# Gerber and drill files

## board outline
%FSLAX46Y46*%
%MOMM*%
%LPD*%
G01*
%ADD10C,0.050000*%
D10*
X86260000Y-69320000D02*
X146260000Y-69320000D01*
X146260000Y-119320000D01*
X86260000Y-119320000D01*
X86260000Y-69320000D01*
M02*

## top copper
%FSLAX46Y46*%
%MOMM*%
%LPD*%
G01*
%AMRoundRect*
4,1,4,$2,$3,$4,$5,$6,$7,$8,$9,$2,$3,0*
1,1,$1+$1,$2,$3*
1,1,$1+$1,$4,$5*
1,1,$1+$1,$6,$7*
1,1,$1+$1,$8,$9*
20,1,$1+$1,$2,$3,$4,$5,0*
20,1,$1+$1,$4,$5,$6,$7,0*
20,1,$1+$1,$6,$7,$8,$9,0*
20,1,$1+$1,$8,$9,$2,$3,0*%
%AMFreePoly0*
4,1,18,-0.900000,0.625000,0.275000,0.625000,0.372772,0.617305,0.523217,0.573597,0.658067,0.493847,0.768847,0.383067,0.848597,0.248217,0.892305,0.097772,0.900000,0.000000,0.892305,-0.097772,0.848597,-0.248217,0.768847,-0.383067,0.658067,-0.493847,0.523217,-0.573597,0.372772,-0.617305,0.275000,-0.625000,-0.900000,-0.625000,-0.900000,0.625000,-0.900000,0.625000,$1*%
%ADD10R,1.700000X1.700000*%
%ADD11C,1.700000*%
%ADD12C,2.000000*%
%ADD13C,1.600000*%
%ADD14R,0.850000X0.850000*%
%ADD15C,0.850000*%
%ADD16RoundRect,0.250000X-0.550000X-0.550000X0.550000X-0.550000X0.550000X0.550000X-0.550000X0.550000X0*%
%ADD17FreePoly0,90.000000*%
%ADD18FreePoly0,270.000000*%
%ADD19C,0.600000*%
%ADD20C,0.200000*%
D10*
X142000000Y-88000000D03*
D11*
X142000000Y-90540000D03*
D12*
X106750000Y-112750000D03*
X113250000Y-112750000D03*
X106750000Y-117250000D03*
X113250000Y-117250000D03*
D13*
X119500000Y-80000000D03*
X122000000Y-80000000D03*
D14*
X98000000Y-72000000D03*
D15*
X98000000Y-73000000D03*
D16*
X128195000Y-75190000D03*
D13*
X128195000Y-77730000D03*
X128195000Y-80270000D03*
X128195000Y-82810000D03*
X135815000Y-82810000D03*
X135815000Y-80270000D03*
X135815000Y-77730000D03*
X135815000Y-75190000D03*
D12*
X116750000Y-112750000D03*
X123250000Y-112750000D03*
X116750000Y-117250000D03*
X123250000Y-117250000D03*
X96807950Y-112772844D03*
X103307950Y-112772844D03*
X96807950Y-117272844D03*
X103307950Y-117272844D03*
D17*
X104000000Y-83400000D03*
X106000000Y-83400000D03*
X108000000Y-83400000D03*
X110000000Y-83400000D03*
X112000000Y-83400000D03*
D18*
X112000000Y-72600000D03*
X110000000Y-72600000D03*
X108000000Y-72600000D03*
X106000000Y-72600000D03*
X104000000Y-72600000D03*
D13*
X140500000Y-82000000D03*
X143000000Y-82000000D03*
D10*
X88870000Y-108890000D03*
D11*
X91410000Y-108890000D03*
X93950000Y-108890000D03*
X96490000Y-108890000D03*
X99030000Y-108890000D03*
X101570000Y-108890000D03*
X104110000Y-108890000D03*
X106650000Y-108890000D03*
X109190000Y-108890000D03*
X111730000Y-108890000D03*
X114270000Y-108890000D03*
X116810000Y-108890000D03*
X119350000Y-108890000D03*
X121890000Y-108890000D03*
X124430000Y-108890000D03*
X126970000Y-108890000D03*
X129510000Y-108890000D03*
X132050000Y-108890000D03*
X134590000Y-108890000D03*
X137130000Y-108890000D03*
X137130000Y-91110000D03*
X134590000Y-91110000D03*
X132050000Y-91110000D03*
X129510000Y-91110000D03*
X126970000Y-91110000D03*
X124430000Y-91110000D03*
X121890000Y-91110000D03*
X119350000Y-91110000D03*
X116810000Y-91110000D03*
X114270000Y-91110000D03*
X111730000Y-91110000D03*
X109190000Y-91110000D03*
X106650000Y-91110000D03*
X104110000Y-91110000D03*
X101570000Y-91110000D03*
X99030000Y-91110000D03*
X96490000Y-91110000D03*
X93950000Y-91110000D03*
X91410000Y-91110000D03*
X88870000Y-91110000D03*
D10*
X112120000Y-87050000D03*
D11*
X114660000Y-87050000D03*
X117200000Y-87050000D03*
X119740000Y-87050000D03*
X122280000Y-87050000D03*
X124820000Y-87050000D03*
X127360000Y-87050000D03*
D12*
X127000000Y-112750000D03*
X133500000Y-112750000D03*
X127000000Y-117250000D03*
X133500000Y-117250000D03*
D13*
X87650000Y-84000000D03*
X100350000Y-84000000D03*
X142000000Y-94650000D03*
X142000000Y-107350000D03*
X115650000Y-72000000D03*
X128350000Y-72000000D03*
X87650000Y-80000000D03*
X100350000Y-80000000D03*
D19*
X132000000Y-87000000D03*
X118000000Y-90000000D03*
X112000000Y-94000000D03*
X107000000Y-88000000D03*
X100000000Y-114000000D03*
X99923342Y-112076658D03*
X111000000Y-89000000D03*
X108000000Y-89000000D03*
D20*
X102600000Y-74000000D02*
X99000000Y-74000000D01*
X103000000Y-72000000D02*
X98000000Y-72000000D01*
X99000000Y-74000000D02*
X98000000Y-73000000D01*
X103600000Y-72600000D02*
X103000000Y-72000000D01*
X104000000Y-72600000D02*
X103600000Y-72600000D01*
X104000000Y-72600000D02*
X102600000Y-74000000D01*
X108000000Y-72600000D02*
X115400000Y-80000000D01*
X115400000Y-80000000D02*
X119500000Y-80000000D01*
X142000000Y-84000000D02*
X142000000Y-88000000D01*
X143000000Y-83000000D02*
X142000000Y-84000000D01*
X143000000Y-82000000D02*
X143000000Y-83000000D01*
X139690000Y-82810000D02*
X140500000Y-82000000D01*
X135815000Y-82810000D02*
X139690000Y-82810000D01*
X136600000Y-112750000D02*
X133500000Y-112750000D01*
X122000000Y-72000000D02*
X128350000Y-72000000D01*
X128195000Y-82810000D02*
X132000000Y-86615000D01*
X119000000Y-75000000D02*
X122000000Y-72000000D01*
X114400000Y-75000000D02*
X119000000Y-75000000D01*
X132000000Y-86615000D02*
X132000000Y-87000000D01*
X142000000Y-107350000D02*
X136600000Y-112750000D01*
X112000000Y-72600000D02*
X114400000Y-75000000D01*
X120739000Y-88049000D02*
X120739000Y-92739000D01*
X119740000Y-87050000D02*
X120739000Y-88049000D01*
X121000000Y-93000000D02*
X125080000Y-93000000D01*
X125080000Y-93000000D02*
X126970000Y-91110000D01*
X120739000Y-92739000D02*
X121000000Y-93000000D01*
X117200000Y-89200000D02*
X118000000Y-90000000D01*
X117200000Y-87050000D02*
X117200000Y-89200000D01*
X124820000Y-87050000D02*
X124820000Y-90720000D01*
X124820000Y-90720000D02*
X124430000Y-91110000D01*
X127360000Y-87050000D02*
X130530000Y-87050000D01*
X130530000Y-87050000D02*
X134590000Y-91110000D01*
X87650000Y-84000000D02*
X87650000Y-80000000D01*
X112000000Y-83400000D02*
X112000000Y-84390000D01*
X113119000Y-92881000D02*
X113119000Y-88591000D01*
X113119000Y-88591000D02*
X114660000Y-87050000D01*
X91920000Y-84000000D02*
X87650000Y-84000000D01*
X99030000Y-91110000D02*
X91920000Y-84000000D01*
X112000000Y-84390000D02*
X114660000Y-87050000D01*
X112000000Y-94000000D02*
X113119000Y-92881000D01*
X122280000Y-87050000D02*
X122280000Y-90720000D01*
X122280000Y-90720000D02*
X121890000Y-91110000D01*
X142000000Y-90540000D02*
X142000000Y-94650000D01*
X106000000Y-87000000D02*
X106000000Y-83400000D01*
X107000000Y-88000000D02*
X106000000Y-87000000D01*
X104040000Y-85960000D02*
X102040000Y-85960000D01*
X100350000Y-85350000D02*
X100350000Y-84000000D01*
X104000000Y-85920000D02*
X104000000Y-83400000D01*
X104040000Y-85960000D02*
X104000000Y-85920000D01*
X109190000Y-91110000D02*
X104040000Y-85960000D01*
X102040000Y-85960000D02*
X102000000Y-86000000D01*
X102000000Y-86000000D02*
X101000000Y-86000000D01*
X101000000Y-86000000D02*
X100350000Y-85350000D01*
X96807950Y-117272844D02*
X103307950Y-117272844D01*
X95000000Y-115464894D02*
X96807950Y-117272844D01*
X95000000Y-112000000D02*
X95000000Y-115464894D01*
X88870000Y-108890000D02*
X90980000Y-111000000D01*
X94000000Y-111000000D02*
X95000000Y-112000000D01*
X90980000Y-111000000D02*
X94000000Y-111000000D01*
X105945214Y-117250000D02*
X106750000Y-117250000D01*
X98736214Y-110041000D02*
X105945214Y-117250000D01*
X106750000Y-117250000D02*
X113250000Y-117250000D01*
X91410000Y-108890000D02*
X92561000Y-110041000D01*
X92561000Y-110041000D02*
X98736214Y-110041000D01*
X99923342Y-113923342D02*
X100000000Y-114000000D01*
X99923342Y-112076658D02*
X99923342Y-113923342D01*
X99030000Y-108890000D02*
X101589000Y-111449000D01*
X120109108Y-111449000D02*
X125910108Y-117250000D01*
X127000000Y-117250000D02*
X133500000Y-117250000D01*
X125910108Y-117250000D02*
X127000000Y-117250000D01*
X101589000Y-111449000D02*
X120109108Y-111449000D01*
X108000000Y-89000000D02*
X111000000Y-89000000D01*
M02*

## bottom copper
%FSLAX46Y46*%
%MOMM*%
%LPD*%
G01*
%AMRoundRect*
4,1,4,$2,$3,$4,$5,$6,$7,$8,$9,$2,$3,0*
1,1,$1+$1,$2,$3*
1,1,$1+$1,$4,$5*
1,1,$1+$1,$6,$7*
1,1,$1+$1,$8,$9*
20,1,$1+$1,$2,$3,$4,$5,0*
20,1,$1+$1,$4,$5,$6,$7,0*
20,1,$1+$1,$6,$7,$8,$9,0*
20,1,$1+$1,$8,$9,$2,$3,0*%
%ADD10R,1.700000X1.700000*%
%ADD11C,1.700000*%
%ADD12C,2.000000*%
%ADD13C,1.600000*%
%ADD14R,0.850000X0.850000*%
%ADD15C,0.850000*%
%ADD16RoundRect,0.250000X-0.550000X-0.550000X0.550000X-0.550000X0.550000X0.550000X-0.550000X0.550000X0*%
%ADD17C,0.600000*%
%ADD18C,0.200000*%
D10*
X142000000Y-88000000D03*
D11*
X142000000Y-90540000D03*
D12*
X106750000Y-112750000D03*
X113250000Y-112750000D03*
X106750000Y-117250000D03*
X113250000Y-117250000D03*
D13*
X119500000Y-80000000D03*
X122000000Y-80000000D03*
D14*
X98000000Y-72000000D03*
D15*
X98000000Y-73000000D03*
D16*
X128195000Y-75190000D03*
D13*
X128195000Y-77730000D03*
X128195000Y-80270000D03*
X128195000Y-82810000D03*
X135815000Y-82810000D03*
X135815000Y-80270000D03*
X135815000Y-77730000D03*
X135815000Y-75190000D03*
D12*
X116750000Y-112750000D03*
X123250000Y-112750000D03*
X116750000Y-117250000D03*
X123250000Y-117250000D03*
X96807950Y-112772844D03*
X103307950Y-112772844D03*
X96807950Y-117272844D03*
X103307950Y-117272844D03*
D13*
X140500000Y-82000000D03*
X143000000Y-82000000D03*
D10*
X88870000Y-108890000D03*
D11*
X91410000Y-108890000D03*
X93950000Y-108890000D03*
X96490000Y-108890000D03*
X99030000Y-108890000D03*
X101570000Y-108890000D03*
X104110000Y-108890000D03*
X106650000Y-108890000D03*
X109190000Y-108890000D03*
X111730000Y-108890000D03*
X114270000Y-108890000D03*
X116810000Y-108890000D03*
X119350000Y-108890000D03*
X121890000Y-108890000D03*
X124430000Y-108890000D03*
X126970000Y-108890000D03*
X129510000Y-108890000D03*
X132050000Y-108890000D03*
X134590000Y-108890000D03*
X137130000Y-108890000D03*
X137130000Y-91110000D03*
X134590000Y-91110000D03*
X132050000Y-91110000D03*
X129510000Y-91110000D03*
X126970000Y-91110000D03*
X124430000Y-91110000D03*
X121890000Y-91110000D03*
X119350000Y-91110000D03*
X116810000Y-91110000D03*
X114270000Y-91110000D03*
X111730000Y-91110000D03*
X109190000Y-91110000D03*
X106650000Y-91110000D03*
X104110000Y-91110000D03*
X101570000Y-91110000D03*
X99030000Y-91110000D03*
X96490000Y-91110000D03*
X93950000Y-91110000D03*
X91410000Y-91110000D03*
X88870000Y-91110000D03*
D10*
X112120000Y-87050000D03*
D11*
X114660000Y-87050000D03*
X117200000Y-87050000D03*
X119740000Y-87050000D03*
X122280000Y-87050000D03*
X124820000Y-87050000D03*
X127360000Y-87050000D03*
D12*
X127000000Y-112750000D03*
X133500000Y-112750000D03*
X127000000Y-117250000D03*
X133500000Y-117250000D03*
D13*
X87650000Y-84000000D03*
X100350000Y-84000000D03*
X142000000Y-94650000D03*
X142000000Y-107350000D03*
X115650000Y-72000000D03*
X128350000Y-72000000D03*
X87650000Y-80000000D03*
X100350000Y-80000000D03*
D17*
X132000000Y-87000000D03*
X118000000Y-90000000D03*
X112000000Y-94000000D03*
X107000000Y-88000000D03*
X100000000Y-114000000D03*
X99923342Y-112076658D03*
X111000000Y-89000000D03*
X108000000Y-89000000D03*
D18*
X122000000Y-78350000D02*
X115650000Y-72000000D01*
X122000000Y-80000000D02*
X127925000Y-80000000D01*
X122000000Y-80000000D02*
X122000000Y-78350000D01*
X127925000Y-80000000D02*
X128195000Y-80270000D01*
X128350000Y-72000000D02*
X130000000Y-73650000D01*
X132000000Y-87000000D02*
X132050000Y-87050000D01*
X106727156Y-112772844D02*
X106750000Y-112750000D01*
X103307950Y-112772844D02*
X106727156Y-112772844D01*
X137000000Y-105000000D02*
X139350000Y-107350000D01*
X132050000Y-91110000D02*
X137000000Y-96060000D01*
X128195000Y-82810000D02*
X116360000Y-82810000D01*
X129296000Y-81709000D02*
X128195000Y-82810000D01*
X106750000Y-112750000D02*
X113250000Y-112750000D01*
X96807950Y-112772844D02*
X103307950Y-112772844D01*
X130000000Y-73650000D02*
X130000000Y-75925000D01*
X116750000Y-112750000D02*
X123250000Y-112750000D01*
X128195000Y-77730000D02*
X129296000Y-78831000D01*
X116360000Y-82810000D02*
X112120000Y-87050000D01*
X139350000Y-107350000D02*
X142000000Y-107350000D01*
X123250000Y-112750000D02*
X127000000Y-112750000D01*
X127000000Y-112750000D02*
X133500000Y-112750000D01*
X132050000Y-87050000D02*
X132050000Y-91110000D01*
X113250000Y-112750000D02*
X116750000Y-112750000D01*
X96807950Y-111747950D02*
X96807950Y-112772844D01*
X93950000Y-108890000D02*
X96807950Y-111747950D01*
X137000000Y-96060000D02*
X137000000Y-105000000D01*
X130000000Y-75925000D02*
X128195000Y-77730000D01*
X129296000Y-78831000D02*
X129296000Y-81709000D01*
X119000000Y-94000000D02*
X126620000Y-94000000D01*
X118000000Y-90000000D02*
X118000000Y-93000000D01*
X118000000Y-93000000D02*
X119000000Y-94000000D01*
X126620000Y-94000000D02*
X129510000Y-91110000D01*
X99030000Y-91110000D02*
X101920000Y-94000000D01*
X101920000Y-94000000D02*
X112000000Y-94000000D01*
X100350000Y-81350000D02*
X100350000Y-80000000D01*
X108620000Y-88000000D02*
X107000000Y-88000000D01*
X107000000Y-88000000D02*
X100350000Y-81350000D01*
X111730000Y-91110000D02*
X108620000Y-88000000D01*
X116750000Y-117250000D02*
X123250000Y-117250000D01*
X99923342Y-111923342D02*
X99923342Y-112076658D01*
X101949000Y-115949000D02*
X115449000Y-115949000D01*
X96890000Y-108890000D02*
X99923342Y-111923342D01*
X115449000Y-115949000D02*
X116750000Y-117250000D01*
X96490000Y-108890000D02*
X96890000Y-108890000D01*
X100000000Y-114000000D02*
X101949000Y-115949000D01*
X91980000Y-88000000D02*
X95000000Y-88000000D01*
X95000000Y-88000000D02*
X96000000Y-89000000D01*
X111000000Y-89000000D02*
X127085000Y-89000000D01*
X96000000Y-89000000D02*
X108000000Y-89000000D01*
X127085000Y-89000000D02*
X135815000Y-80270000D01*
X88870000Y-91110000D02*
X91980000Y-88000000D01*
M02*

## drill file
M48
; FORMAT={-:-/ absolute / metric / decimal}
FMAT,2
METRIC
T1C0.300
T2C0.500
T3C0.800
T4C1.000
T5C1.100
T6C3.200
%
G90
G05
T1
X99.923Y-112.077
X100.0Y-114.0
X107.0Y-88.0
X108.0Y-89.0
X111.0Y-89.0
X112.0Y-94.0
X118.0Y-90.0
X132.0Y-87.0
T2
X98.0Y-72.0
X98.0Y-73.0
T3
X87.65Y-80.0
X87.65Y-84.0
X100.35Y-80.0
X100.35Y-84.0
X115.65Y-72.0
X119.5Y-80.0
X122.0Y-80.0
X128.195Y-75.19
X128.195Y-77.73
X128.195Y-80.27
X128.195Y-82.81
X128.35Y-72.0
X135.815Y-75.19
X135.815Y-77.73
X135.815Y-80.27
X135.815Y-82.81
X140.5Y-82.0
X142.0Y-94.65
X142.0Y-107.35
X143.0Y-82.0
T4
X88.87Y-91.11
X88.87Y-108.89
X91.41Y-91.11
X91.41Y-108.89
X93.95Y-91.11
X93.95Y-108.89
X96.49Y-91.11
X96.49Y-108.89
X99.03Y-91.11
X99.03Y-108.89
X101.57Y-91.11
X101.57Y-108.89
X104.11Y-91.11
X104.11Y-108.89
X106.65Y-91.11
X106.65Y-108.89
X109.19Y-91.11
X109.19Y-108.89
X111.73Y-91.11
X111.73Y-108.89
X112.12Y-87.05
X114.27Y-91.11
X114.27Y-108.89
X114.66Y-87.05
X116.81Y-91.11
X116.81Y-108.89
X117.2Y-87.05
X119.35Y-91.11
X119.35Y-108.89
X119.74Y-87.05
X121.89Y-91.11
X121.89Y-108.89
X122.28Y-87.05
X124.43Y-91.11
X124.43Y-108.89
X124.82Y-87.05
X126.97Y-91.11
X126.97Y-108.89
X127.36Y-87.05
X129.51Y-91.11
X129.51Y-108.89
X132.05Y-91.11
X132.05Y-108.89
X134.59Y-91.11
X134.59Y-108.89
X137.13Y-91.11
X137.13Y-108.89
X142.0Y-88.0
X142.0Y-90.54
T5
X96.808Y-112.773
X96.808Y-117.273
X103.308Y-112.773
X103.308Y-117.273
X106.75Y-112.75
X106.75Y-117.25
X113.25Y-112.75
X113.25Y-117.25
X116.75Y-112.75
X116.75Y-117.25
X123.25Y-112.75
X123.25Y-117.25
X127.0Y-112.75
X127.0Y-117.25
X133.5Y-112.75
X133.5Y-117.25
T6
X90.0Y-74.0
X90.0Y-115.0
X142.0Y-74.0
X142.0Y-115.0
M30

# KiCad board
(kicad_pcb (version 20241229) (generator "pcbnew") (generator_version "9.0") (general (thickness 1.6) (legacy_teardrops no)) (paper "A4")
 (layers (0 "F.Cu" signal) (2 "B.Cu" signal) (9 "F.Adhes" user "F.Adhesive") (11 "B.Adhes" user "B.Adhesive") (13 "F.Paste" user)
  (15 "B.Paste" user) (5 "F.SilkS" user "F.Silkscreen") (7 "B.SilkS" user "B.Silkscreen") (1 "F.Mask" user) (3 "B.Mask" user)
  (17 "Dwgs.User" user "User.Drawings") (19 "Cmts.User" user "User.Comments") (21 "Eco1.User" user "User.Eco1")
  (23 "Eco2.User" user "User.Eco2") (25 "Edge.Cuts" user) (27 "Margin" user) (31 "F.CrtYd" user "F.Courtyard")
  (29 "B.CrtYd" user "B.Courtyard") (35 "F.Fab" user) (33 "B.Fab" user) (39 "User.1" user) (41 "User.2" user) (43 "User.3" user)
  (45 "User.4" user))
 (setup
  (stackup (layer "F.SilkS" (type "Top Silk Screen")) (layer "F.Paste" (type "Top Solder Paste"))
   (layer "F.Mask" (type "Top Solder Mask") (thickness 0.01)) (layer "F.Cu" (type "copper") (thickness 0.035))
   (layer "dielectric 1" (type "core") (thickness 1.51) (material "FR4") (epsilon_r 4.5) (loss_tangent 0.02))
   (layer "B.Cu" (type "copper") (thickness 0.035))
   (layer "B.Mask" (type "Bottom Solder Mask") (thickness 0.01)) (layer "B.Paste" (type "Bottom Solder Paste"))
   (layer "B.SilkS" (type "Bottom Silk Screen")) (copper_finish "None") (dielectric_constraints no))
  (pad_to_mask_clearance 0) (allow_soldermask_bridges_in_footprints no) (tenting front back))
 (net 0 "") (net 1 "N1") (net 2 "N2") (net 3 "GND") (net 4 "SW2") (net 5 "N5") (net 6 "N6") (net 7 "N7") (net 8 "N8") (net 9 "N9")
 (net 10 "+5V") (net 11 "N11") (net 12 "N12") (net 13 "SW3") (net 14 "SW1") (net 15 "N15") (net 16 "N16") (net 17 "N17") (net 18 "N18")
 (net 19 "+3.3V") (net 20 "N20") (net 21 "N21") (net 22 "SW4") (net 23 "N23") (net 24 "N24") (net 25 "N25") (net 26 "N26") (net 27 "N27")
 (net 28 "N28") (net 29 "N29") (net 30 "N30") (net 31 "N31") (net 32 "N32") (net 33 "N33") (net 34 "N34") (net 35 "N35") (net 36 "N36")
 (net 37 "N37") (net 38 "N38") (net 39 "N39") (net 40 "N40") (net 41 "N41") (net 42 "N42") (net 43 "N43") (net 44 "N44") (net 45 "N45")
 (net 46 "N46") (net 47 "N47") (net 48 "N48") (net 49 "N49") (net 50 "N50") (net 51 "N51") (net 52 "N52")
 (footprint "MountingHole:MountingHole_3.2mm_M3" (layer "F.Cu") (at 90 115)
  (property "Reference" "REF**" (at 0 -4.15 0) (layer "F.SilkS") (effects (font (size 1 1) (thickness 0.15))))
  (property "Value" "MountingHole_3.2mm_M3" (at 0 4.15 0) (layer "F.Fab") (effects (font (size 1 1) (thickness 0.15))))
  (pad "" np_thru_hole circle (at 0 0) (size 3.2 3.2) (drill 3.2) (layers "*.Cu" "*.Mask")))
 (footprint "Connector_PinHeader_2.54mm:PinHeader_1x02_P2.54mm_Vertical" (layer "F.Cu") (at 142 88)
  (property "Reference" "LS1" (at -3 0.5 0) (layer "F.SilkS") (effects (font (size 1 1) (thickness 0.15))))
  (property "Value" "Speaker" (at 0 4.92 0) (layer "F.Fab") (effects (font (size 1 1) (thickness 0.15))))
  (pad "1" thru_hole rect (at 0 0) (size 1.7 1.7) (drill 1) (layers "*.Cu" "*.Mask") (remove_unused_layers no) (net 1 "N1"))
  (pad "2" thru_hole circle (at 0 2.54) (size 1.7 1.7) (drill 1) (layers "*.Cu" "*.Mask") (remove_unused_layers no) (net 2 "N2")))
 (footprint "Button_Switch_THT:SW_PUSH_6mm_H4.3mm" (layer "F.Cu") (at 106.75 112.75)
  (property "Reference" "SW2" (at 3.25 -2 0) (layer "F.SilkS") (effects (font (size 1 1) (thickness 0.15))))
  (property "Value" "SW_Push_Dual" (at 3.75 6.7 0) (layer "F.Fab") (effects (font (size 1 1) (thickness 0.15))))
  (pad "1" thru_hole circle (at 0 0 90) (size 2 2) (drill 1.1) (layers "*.Cu" "*.Mask") (remove_unused_layers no) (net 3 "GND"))
  (pad "1" thru_hole circle (at 6.5 0 90) (size 2 2) (drill 1.1) (layers "*.Cu" "*.Mask") (remove_unused_layers no) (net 3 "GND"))
  (pad "2" thru_hole circle (at 0 4.5 90) (size 2 2) (drill 1.1) (layers "*.Cu" "*.Mask") (remove_unused_layers no) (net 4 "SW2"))
  (pad "2" thru_hole circle (at 6.5 4.5 90) (size 2 2) (drill 1.1) (layers "*.Cu" "*.Mask") (remove_unused_layers no) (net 4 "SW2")))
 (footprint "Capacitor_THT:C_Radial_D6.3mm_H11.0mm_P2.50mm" (layer "F.Cu") (at 119.5 80)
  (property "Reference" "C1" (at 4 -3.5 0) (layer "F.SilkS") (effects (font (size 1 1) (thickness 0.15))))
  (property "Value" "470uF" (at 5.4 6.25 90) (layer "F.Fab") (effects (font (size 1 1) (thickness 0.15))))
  (pad "1" thru_hole circle (at 0 0) (size 1.6 1.6) (drill 0.8) (layers "*.Cu" "*.Mask") (remove_unused_layers no) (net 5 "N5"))
  (pad "2" thru_hole circle (at 2.5 0) (size 1.6 1.6) (drill 0.8) (layers "*.Cu" "*.Mask") (remove_unused_layers no) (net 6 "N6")))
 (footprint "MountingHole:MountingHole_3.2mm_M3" (layer "F.Cu") (at 142 115)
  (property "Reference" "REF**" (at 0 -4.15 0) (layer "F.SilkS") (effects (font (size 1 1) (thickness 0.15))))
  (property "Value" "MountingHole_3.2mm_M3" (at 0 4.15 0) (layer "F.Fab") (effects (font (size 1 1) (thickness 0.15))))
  (pad "" np_thru_hole circle (at 0 0) (size 3.2 3.2) (drill 3.2) (layers "*.Cu" "*.Mask")))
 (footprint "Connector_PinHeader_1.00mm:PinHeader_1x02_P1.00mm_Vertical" (layer "F.Cu") (at 98 72)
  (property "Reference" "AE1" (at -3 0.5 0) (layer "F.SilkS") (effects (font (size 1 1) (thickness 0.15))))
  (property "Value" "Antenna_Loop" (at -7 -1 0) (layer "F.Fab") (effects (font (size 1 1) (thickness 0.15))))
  (pad "1" thru_hole rect (at 0 0) (size 0.85 0.85) (drill 0.5) (layers "*.Cu" "*.Mask") (remove_unused_layers no) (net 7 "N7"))
  (pad "2" thru_hole circle (at 0 1) (size 0.85 0.85) (drill 0.5) (layers "*.Cu" "*.Mask") (remove_unused_layers no) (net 7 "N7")))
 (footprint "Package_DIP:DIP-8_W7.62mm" (layer "F.Cu") (at 128.195 75.19)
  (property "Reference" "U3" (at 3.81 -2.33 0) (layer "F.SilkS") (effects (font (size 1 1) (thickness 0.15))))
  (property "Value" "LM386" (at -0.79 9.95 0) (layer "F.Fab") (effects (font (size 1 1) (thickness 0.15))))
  (pad "1" thru_hole roundrect (at 0 0) (size 1.6 1.6) (drill 0.8) (layers "*.Cu" "*.Mask") (remove_unused_layers no)
   (roundrect_rratio 0.15625) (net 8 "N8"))
  (pad "2" thru_hole circle (at 0 2.54) (size 1.6 1.6) (drill 0.8) (layers "*.Cu" "*.Mask") (remove_unused_layers no) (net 3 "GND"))
  (pad "3" thru_hole circle (at 0 5.08) (size 1.6 1.6) (drill 0.8) (layers "*.Cu" "*.Mask") (remove_unused_layers no) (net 6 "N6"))
  (pad "4" thru_hole circle (at 0 7.62) (size 1.6 1.6) (drill 0.8) (layers "*.Cu" "*.Mask") (remove_unused_layers no) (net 3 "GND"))
  (pad "5" thru_hole circle (at 7.62 7.62) (size 1.6 1.6) (drill 0.8) (layers "*.Cu" "*.Mask") (remove_unused_layers no) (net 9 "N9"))
  (pad "6" thru_hole circle (at 7.62 5.08) (size 1.6 1.6) (drill 0.8) (layers "*.Cu" "*.Mask") (remove_unused_layers no) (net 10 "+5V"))
  (pad "7" thru_hole circle (at 7.62 2.54) (size 1.6 1.6) (drill 0.8) (layers "*.Cu" "*.Mask") (remove_unused_layers no) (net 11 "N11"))
  (pad "8" thru_hole circle (at 7.62 0) (size 1.6 1.6) (drill 0.8) (layers "*.Cu" "*.Mask") (remove_unused_layers no) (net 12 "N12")))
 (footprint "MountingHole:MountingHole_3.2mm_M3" (layer "F.Cu") (at 142 74)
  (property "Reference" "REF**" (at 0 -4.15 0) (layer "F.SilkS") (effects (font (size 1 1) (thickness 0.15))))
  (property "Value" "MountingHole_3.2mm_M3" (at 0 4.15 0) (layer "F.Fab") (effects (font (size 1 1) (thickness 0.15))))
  (pad "" np_thru_hole circle (at 0 0) (size 3.2 3.2) (drill 3.2) (layers "*.Cu" "*.Mask")))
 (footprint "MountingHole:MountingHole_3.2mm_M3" (layer "F.Cu") (at 90 74)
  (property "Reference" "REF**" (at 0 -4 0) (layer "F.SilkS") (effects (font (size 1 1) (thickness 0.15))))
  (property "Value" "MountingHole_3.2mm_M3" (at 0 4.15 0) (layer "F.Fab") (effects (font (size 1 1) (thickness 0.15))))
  (pad "" np_thru_hole circle (at 0 0) (size 3.2 3.2) (drill 3.2) (layers "*.Cu" "*.Mask")))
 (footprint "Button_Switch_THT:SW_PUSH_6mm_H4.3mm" (layer "F.Cu") (at 116.75 112.75)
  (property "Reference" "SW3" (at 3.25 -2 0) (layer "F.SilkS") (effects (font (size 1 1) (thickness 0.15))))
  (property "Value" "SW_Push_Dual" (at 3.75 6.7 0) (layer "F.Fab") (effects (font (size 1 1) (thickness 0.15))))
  (pad "1" thru_hole circle (at 0 0 90) (size 2 2) (drill 1.1) (layers "*.Cu" "*.Mask") (remove_unused_layers no) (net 3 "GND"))
  (pad "1" thru_hole circle (at 6.5 0 90) (size 2 2) (drill 1.1) (layers "*.Cu" "*.Mask") (remove_unused_layers no) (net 3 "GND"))
  (pad "2" thru_hole circle (at 0 4.5 90) (size 2 2) (drill 1.1) (layers "*.Cu" "*.Mask") (remove_unused_layers no) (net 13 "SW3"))
  (pad "2" thru_hole circle (at 6.5 4.5 90) (size 2 2) (drill 1.1) (layers "*.Cu" "*.Mask") (remove_unused_layers no) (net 13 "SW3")))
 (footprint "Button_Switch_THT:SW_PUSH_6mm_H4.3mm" (layer "F.Cu") (at 96.80795 112.772844)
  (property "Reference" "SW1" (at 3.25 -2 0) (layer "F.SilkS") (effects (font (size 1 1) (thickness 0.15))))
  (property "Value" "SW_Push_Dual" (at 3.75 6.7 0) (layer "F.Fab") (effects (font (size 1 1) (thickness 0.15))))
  (pad "1" thru_hole circle (at 0 0 90) (size 2 2) (drill 1.1) (layers "*.Cu" "*.Mask") (remove_unused_layers no) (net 3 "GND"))
  (pad "1" thru_hole circle (at 6.5 0 90) (size 2 2) (drill 1.1) (layers "*.Cu" "*.Mask") (remove_unused_layers no) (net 3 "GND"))
  (pad "2" thru_hole circle (at 0 4.5 90) (size 2 2) (drill 1.1) (layers "*.Cu" "*.Mask") (remove_unused_layers no) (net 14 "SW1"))
  (pad "2" thru_hole circle (at 6.5 4.5 90) (size 2 2) (drill 1.1) (layers "*.Cu" "*.Mask") (remove_unused_layers no) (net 14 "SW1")))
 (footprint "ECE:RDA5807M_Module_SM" (layer "F.Cu") (at 108 78 90)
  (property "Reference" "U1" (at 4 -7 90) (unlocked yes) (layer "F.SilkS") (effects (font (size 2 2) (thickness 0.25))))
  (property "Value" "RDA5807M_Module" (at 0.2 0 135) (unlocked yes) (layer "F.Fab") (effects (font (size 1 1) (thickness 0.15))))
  (pad "1" smd roundrect (at -5.4 -4 90) (size 1.8 1.25) (layers "F.Cu" "F.Mask" "F.Paste") (roundrect_rratio 0.5) (chamfer_ratio 0)
   (chamfer top_left bottom_left) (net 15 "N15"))
  (pad "2" smd roundrect (at -5.4 -2 90) (size 1.8 1.25) (layers "F.Cu" "F.Mask" "F.Paste") (roundrect_rratio 0.5) (chamfer_ratio 0)
   (chamfer top_left bottom_left) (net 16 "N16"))
  (pad "3" smd roundrect (at -5.4 0 90) (size 1.8 1.25) (layers "F.Cu" "F.Mask" "F.Paste") (roundrect_rratio 0.5) (chamfer_ratio 0)
   (chamfer top_left bottom_left) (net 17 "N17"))
  (pad "4" smd roundrect (at -5.4 2 90) (size 1.8 1.25) (layers "F.Cu" "F.Mask" "F.Paste") (roundrect_rratio 0.5) (chamfer_ratio 0)
   (chamfer top_left bottom_left) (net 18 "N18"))
  (pad "5" smd roundrect (at -5.4 4 90) (size 1.8 1.25) (layers "F.Cu" "F.Mask" "F.Paste") (roundrect_rratio 0.5) (chamfer_ratio 0)
   (chamfer top_left bottom_left) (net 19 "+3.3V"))
  (pad "6" smd roundrect (at 5.4 4 270) (size 1.8 1.25) (layers "F.Cu" "F.Mask" "F.Paste") (roundrect_rratio 0.5) (chamfer_ratio 0)
   (chamfer top_left bottom_left) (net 3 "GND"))
  (pad "7" smd roundrect (at 5.4 2 270) (size 1.8 1.25) (layers "F.Cu" "F.Mask" "F.Paste") (roundrect_rratio 0.5) (chamfer_ratio 0)
   (chamfer top_left bottom_left) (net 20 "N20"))
  (pad "8" smd roundrect (at 5.4 0 270) (size 1.8 1.25) (layers "F.Cu" "F.Mask" "F.Paste") (roundrect_rratio 0.5) (chamfer_ratio 0)
   (chamfer top_left bottom_left) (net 5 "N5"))
  (pad "9" smd roundrect (at 5.4 -2 270) (size 1.8 1.25) (layers "F.Cu" "F.Mask" "F.Paste") (roundrect_rratio 0.5) (chamfer_ratio 0)
   (chamfer top_left bottom_left) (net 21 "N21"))
  (pad "10" smd roundrect (at 5.4 -4 270) (size 1.8 1.25) (layers "F.Cu" "F.Mask" "F.Paste") (roundrect_rratio 0.5) (chamfer_ratio 0)
   (chamfer top_left bottom_left) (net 7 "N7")))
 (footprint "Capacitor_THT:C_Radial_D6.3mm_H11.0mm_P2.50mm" (layer "F.Cu") (at 140.5 82)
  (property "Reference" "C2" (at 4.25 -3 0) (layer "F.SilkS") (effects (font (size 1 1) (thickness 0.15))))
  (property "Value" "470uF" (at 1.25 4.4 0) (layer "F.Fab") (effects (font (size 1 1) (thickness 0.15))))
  (pad "1" thru_hole circle (at 0 0) (size 1.6 1.6) (drill 0.8) (layers "*.Cu" "*.Mask") (remove_unused_layers no) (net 9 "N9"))
  (pad "2" thru_hole circle (at 2.5 0) (size 1.6 1.6) (drill 0.8) (layers "*.Cu" "*.Mask") (remove_unused_layers no) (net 1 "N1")))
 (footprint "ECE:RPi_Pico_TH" (layer "F.Cu") (at 113 100 90)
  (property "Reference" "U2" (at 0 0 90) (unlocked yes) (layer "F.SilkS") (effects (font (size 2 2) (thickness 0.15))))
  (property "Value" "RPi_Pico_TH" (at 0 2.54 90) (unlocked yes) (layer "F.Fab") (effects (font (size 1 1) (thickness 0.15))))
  (pad "1" thru_hole rect (at -8.89 -24.13 90) (size 1.7 1.7) (drill 1) (layers "*.Cu" "*.Mask") (remove_unused_layers no) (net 14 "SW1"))
  (pad "2" thru_hole circle (at -8.89 -21.59 90) (size 1.7 1.7) (drill 1) (layers "*.Cu" "*.Mask") (remove_unused_layers no) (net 4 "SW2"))
  (pad "3" thru_hole circle (at -8.89 -19.05 90) (size 1.7 1.7) (drill 1) (layers "*.Cu" "*.Mask") (remove_unused_layers no) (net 3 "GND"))
  (pad "4" thru_hole circle (at -8.89 -16.51 90) (size 1.7 1.7) (drill 1) (layers "*.Cu" "*.Mask") (remove_unused_layers no) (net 13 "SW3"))
  (pad "5" thru_hole circle (at -8.89 -13.97 90) (size 1.7 1.7) (drill 1) (layers "*.Cu" "*.Mask") (remove_unused_layers no) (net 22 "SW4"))
  (pad "6" thru_hole circle (at -8.89 -11.43 90) (size 1.7 1.7) (drill 1) (layers "*.Cu" "*.Mask") (remove_unused_layers no) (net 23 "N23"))
  (pad "7" thru_hole circle (at -8.89 -8.89 90) (size 1.7 1.7) (drill 1) (layers "*.Cu" "*.Mask") (remove_unused_layers no) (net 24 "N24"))
  (pad "8" thru_hole circle (at -8.89 -6.35 90) (size 1.7 1.7) (drill 1) (layers "*.Cu" "*.Mask") (remove_unused_layers no) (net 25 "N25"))
  (pad "9" thru_hole circle (at -8.89 -3.81 90) (size 1.7 1.7) (drill 1) (layers "*.Cu" "*.Mask") (remove_unused_layers no) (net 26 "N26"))
  (pad "10" thru_hole circle (at -8.89 -1.27 90) (size 1.7 1.7) (drill 1) (layers "*.Cu" "*.Mask") (remove_unused_layers no) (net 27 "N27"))
  (pad "11" thru_hole circle (at -8.89 1.27 90) (size 1.7 1.7) (drill 1) (layers "*.Cu" "*.Mask") (remove_unused_layers no) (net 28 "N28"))
  (pad "12" thru_hole circle (at -8.89 3.81 90) (size 1.7 1.7) (drill 1) (layers "*.Cu" "*.Mask") (remove_unused_layers no) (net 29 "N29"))
  (pad "13" thru_hole circle (at -8.89 6.35 90) (size 1.7 1.7) (drill 1) (layers "*.Cu" "*.Mask") (remove_unused_layers no) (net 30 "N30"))
  (pad "14" thru_hole circle (at -8.89 8.89 90) (size 1.7 1.7) (drill 1) (layers "*.Cu" "*.Mask") (remove_unused_layers no) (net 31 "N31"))
  (pad "15" thru_hole circle (at -8.89 11.43 90) (size 1.7 1.7) (drill 1) (layers "*.Cu" "*.Mask") (remove_unused_layers no) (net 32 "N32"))
  (pad "16" thru_hole circle (at -8.89 13.97 90) (size 1.7 1.7) (drill 1) (layers "*.Cu" "*.Mask") (remove_unused_layers no) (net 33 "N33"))
  (pad "17" thru_hole circle (at -8.89 16.51 90) (size 1.7 1.7) (drill 1) (layers "*.Cu" "*.Mask") (remove_unused_layers no) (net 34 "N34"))
  (pad "18" thru_hole circle (at -8.89 19.05 90) (size 1.7 1.7) (drill 1) (layers "*.Cu" "*.Mask") (remove_unused_layers no) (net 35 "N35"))
  (pad "19" thru_hole circle (at -8.89 21.59 90) (size 1.7 1.7) (drill 1) (layers "*.Cu" "*.Mask") (remove_unused_layers no) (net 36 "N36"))
  (pad "20" thru_hole circle (at -8.89 24.13 90) (size 1.7 1.7) (drill 1) (layers "*.Cu" "*.Mask") (remove_unused_layers no) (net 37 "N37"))
  (pad "21" thru_hole circle (at 8.89 24.13 90) (size 1.7 1.7) (drill 1) (layers "*.Cu" "*.Mask") (remove_unused_layers no) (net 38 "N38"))
  (pad "22" thru_hole circle (at 8.89 21.59 90) (size 1.7 1.7) (drill 1) (layers "*.Cu" "*.Mask") (remove_unused_layers no) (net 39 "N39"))
  (pad "23" thru_hole circle (at 8.89 19.05 90) (size 1.7 1.7) (drill 1) (layers "*.Cu" "*.Mask") (remove_unused_layers no) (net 3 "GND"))
  (pad "24" thru_hole circle (at 8.89 16.51 90) (size 1.7 1.7) (drill 1) (layers "*.Cu" "*.Mask") (remove_unused_layers no) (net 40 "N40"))
  (pad "25" thru_hole circle (at 8.89 13.97 90) (size 1.7 1.7) (drill 1) (layers "*.Cu" "*.Mask") (remove_unused_layers no) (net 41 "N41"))
  (pad "26" thru_hole circle (at 8.89 11.43 90) (size 1.7 1.7) (drill 1) (layers "*.Cu" "*.Mask") (remove_unused_layers no) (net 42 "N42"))
  (pad "27" thru_hole circle (at 8.89 8.89 90) (size 1.7 1.7) (drill 1) (layers "*.Cu" "*.Mask") (remove_unused_layers no) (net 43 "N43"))
  (pad "28" thru_hole circle (at 8.89 6.35 90) (size 1.7 1.7) (drill 1) (layers "*.Cu" "*.Mask") (remove_unused_layers no) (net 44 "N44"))
  (pad "29" thru_hole circle (at 8.89 3.81 90) (size 1.7 1.7) (drill 1) (layers "*.Cu" "*.Mask") (remove_unused_layers no) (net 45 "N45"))
  (pad "30" thru_hole circle (at 8.89 1.27 90) (size 1.7 1.7) (drill 1) (layers "*.Cu" "*.Mask") (remove_unused_layers no) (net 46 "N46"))
  (pad "31" thru_hole circle (at 8.89 -1.27 90) (size 1.7 1.7) (drill 1) (layers "*.Cu" "*.Mask") (remove_unused_layers no) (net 16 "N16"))
  (pad "32" thru_hole circle (at 8.89 -3.81 90) (size 1.7 1.7) (drill 1) (layers "*.Cu" "*.Mask") (remove_unused_layers no) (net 15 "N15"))
  (pad "33" thru_hole circle (at 8.89 -6.35 90) (size 1.7 1.7) (drill 1) (layers "*.Cu" "*.Mask") (remove_unused_layers no) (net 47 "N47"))
  (pad "34" thru_hole circle (at 8.89 -8.89 90) (size 1.7 1.7) (drill 1) (layers "*.Cu" "*.Mask") (remove_unused_layers no) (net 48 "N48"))
  (pad "35" thru_hole circle (at 8.89 -11.43 90) (size 1.7 1.7) (drill 1) (layers "*.Cu" "*.Mask") (remove_unused_layers no) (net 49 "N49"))
  (pad "36" thru_hole circle (at 8.89 -13.97 90) (size 1.7 1.7) (drill 1) (layers "*.Cu" "*.Mask") (remove_unused_layers no)
   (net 19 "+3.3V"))
  (pad "37" thru_hole circle (at 8.89 -16.51 90) (size 1.7 1.7) (drill 1) (layers "*.Cu" "*.Mask") (remove_unused_layers no) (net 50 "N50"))
  (pad "38" thru_hole circle (at 8.89 -19.05 90) (size 1.7 1.7) (drill 1) (layers "*.Cu" "*.Mask") (remove_unused_layers no) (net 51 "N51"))
  (pad "39" thru_hole circle (at 8.89 -21.59 90) (size 1.7 1.7) (drill 1) (layers "*.Cu" "*.Mask") (remove_unused_layers no) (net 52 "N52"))
  (pad "40" thru_hole circle (at 8.89 -24.13 90) (size 1.7 1.7) (drill 1) (layers "*.Cu" "*.Mask") (remove_unused_layers no) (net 10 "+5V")))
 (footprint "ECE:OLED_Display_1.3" (layer "F.Cu") (at 102 119)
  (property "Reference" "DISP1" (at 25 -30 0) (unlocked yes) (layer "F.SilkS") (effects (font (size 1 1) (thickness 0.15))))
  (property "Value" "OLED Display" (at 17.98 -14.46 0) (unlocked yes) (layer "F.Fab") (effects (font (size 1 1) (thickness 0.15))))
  (pad "1" thru_hole rect (at 10.12 -31.95 270) (size 1.7 1.7) (drill 1) (layers "*.Cu" "*.Mask") (remove_unused_layers no) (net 3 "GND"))
  (pad "2" thru_hole circle (at 12.66 -31.95 270) (size 1.7 1.7) (drill 1) (layers "*.Cu" "*.Mask") (remove_unused_layers no)
   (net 19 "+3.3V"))
  (pad "3" thru_hole circle (at 15.2 -31.95 270) (size 1.7 1.7) (drill 1) (layers "*.Cu" "*.Mask") (remove_unused_layers no) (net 40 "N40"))
  (pad "4" thru_hole circle (at 17.74 -31.95 270) (size 1.7 1.7) (drill 1) (layers "*.Cu" "*.Mask") (remove_unused_layers no) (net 41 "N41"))
  (pad "5" thru_hole circle (at 20.28 -31.95 270) (size 1.7 1.7) (drill 1) (layers "*.Cu" "*.Mask") (remove_unused_layers no) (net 43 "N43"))
  (pad "6" thru_hole circle (at 22.82 -31.95 270) (size 1.7 1.7) (drill 1) (layers "*.Cu" "*.Mask") (remove_unused_layers no) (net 42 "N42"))
  (pad "7" thru_hole circle (at 25.36 -31.95 270) (size 1.7 1.7) (drill 1) (layers "*.Cu" "*.Mask") (remove_unused_layers no) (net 39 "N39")))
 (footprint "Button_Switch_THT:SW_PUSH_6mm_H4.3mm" (layer "F.Cu") (at 127 112.75)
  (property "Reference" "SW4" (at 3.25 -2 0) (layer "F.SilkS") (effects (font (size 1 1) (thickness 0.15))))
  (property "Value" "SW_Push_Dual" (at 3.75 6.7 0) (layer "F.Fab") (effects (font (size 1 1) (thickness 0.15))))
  (pad "1" thru_hole circle (at 0 0 90) (size 2 2) (drill 1.1) (layers "*.Cu" "*.Mask") (remove_unused_layers no) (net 3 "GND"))
  (pad "1" thru_hole circle (at 6.5 0 90) (size 2 2) (drill 1.1) (layers "*.Cu" "*.Mask") (remove_unused_layers no) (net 3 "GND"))
  (pad "2" thru_hole circle (at 0 4.5 90) (size 2 2) (drill 1.1) (layers "*.Cu" "*.Mask") (remove_unused_layers no) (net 22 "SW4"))
  (pad "2" thru_hole circle (at 6.5 4.5 90) (size 2 2) (drill 1.1) (layers "*.Cu" "*.Mask") (remove_unused_layers no) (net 22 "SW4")))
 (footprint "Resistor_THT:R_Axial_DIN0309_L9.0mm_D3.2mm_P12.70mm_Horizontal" (layer "B.Cu") (at 87.65 84)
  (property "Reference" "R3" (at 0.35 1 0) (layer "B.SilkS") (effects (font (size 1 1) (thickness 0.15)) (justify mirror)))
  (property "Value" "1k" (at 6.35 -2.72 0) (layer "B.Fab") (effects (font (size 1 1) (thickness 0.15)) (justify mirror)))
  (pad "1" thru_hole circle (at 0 0) (size 1.6 1.6) (drill 0.8) (layers "*.Cu" "*.Mask") (remove_unused_layers no) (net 19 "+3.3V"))
  (pad "2" thru_hole circle (at 12.7 0) (size 1.6 1.6) (drill 0.8) (layers "*.Cu" "*.Mask") (remove_unused_layers no) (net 15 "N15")))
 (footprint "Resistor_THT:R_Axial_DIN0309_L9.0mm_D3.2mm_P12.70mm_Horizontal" (layer "B.Cu") (at 142 94.65 -90)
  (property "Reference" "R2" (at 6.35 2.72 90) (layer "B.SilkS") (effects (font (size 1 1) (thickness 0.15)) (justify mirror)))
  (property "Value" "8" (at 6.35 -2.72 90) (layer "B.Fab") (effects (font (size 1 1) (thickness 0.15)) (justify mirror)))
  (pad "1" thru_hole circle (at 0 0 270) (size 1.6 1.6) (drill 0.8) (layers "*.Cu" "*.Mask") (remove_unused_layers no) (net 2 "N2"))
  (pad "2" thru_hole circle (at 12.7 0 270) (size 1.6 1.6) (drill 0.8) (layers "*.Cu" "*.Mask") (remove_unused_layers no) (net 3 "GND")))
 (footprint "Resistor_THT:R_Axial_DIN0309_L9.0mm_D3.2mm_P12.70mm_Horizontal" (layer "B.Cu") (at 115.65 72)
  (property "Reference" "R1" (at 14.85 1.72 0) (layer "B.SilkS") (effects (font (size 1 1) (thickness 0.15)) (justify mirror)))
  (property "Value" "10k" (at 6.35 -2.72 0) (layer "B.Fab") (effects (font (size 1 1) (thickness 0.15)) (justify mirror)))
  (pad "1" thru_hole circle (at 0 0) (size 1.6 1.6) (drill 0.8) (layers "*.Cu" "*.Mask") (remove_unused_layers no) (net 6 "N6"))
  (pad "2" thru_hole circle (at 12.7 0) (size 1.6 1.6) (drill 0.8) (layers "*.Cu" "*.Mask") (remove_unused_layers no) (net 3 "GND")))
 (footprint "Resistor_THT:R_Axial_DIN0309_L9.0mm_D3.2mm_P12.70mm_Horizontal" (layer "B.Cu") (at 87.65 80)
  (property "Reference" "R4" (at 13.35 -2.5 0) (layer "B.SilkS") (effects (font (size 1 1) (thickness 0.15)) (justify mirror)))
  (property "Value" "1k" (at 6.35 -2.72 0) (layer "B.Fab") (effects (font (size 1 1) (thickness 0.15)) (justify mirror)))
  (pad "1" thru_hole circle (at 0 0) (size 1.6 1.6) (drill 0.8) (layers "*.Cu" "*.Mask") (remove_unused_layers no) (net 19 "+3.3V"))
  (pad "2" thru_hole circle (at 12.7 0) (size 1.6 1.6) (drill 0.8) (layers "*.Cu" "*.Mask") (remove_unused_layers no) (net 16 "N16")))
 (gr_rect (start 86.26 69.32) (end 146.26 119.32) (stroke (width 0.05) (type default)) (fill no) (layer "Edge.Cuts"))
 (segment (start 102.6 74) (end 99 74) (width 0.2) (layer "F.Cu") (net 7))
 (segment (start 103 72) (end 98 72) (width 0.2) (layer "F.Cu") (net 7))
 (segment (start 99 74) (end 98 73) (width 0.2) (layer "F.Cu") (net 7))
 (segment (start 103.6 72.6) (end 103 72) (width 0.2) (layer "F.Cu") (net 7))
 (segment (start 104 72.6) (end 103.6 72.6) (width 0.2) (layer "F.Cu") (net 7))
 (segment (start 104 72.6) (end 102.6 74) (width 0.2) (layer "F.Cu") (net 7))
 (segment (start 122 78.35) (end 115.65 72) (width 0.2) (layer "B.Cu") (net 6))
 (segment (start 122 80) (end 127.925 80) (width 0.2) (layer "B.Cu") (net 6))
 (segment (start 122 80) (end 122 78.35) (width 0.2) (layer "B.Cu") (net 6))
 (segment (start 127.925 80) (end 128.195 80.27) (width 0.2) (layer "B.Cu") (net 6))
 (segment (start 108 72.6) (end 115.4 80) (width 0.2) (layer "F.Cu") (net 5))
 (segment (start 115.4 80) (end 119.5 80) (width 0.2) (layer "F.Cu") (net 5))
 (segment (start 142 84) (end 142 88) (width 0.2) (layer "F.Cu") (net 1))
 (segment (start 143 83) (end 142 84) (width 0.2) (layer "F.Cu") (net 1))
 (segment (start 143 82) (end 143 83) (width 0.2) (layer "F.Cu") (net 1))
 (segment (start 139.69 82.81) (end 140.5 82) (width 0.2) (layer "F.Cu") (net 9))
 (segment (start 135.815 82.81) (end 139.69 82.81) (width 0.2) (layer "F.Cu") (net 9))
 (segment (start 136.6 112.75) (end 133.5 112.75) (width 0.2) (layer "F.Cu") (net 3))
 (segment (start 122 72) (end 128.35 72) (width 0.2) (layer "F.Cu") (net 3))
 (segment (start 128.195 82.81) (end 132 86.615) (width 0.2) (layer "F.Cu") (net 3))
 (segment (start 119 75) (end 122 72) (width 0.2) (layer "F.Cu") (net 3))
 (segment (start 114.4 75) (end 119 75) (width 0.2) (layer "F.Cu") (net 3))
 (segment (start 132 86.615) (end 132 87) (width 0.2) (layer "F.Cu") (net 3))
 (segment (start 142 107.35) (end 136.6 112.75) (width 0.2) (layer "F.Cu") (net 3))
 (segment (start 112 72.6) (end 114.4 75) (width 0.2) (layer "F.Cu") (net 3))
 (via (at 132 87) (size 0.6) (drill 0.3) (layers "F.Cu" "B.Cu") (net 3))
 (segment (start 128.35 72) (end 130 73.65) (width 0.2) (layer "B.Cu") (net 3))
 (segment (start 132 87) (end 132.05 87.05) (width 0.2) (layer "B.Cu") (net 3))
 (segment (start 106.727156 112.772844) (end 106.75 112.75) (width 0.2) (layer "B.Cu") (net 3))
 (segment (start 103.30795 112.772844) (end 106.727156 112.772844) (width 0.2) (layer "B.Cu") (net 3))
 (segment (start 137 105) (end 139.35 107.35) (width 0.2) (layer "B.Cu") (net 3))
 (segment (start 132.05 91.11) (end 137 96.06) (width 0.2) (layer "B.Cu") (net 3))
 (segment (start 128.195 82.81) (end 116.36 82.81) (width 0.2) (layer "B.Cu") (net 3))
 (segment (start 129.296 81.709) (end 128.195 82.81) (width 0.2) (layer "B.Cu") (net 3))
 (segment (start 106.75 112.75) (end 113.25 112.75) (width 0.2) (layer "B.Cu") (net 3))
 (segment (start 96.80795 112.772844) (end 103.30795 112.772844) (width 0.2) (layer "B.Cu") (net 3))
 (segment (start 130 73.65) (end 130 75.925) (width 0.2) (layer "B.Cu") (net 3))
 (segment (start 116.75 112.75) (end 123.25 112.75) (width 0.2) (layer "B.Cu") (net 3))
 (segment (start 128.195 77.73) (end 129.296 78.831) (width 0.2) (layer "B.Cu") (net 3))
 (segment (start 116.36 82.81) (end 112.12 87.05) (width 0.2) (layer "B.Cu") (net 3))
 (segment (start 139.35 107.35) (end 142 107.35) (width 0.2) (layer "B.Cu") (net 3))
 (segment (start 123.25 112.75) (end 127 112.75) (width 0.2) (layer "B.Cu") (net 3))
 (segment (start 127 112.75) (end 133.5 112.75) (width 0.2) (layer "B.Cu") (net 3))
 (segment (start 132.05 87.05) (end 132.05 91.11) (width 0.2) (layer "B.Cu") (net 3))
 (segment (start 113.25 112.75) (end 116.75 112.75) (width 0.2) (layer "B.Cu") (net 3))
 (segment (start 96.80795 111.74795) (end 96.80795 112.772844) (width 0.2) (layer "B.Cu") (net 3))
 (segment (start 93.95 108.89) (end 96.80795 111.74795) (width 0.2) (layer "B.Cu") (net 3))
 (segment (start 137 96.06) (end 137 105) (width 0.2) (layer "B.Cu") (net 3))
 (segment (start 130 75.925) (end 128.195 77.73) (width 0.2) (layer "B.Cu") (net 3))
 (segment (start 129.296 78.831) (end 129.296 81.709) (width 0.2) (layer "B.Cu") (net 3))
 (segment (start 120.739 88.049) (end 120.739 92.739) (width 0.2) (layer "F.Cu") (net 41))
 (segment (start 119.74 87.05) (end 120.739 88.049) (width 0.2) (layer "F.Cu") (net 41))
 (segment (start 121 93) (end 125.08 93) (width 0.2) (layer "F.Cu") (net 41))
 (segment (start 125.08 93) (end 126.97 91.11) (width 0.2) (layer "F.Cu") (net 41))
 (segment (start 120.739 92.739) (end 121 93) (width 0.2) (layer "F.Cu") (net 41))
 (segment (start 117.2 89.2) (end 118 90) (width 0.2) (layer "F.Cu") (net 40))
 (segment (start 117.2 87.05) (end 117.2 89.2) (width 0.2) (layer "F.Cu") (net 40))
 (via (at 118 90) (size 0.6) (drill 0.3) (layers "F.Cu" "B.Cu") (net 40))
 (segment (start 119 94) (end 126.62 94) (width 0.2) (layer "B.Cu") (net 40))
 (segment (start 118 90) (end 118 93) (width 0.2) (layer "B.Cu") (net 40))
 (segment (start 118 93) (end 119 94) (width 0.2) (layer "B.Cu") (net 40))
 (segment (start 126.62 94) (end 129.51 91.11) (width 0.2) (layer "B.Cu") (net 40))
 (segment (start 124.82 87.05) (end 124.82 90.72) (width 0.2) (layer "F.Cu") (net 42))
 (segment (start 124.82 90.72) (end 124.43 91.11) (width 0.2) (layer "F.Cu") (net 42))
 (segment (start 127.36 87.05) (end 130.53 87.05) (width 0.2) (layer "F.Cu") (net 39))
 (segment (start 130.53 87.05) (end 134.59 91.11) (width 0.2) (layer "F.Cu") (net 39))
 (segment (start 87.65 84) (end 87.65 80) (width 0.2) (layer "F.Cu") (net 19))
 (segment (start 112 83.4) (end 112 84.39) (width 0.2) (layer "F.Cu") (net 19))
 (segment (start 113.119 92.881) (end 113.119 88.591) (width 0.2) (layer "F.Cu") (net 19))
 (segment (start 113.119 88.591) (end 114.66 87.05) (width 0.2) (layer "F.Cu") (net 19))
 (segment (start 91.92 84) (end 87.65 84) (width 0.2) (layer "F.Cu") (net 19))
 (segment (start 99.03 91.11) (end 91.92 84) (width 0.2) (layer "F.Cu") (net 19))
 (segment (start 112 84.39) (end 114.66 87.05) (width 0.2) (layer "F.Cu") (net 19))
 (segment (start 112 94) (end 113.119 92.881) (width 0.2) (layer "F.Cu") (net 19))
 (via (at 112 94) (size 0.6) (drill 0.3) (layers "F.Cu" "B.Cu") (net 19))
 (segment (start 99.03 91.11) (end 101.92 94) (width 0.2) (layer "B.Cu") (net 19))
 (segment (start 101.92 94) (end 112 94) (width 0.2) (layer "B.Cu") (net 19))
 (segment (start 122.28 87.05) (end 122.28 90.72) (width 0.2) (layer "F.Cu") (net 43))
 (segment (start 122.28 90.72) (end 121.89 91.11) (width 0.2) (layer "F.Cu") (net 43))
 (segment (start 142 90.54) (end 142 94.65) (width 0.2) (layer "F.Cu") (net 2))
 (segment (start 106 87) (end 106 83.4) (width 0.2) (layer "F.Cu") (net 16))
 (segment (start 107 88) (end 106 87) (width 0.2) (layer "F.Cu") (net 16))
 (via (at 107 88) (size 0.6) (drill 0.3) (layers "F.Cu" "B.Cu") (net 16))
 (segment (start 100.35 81.35) (end 100.35 80) (width 0.2) (layer "B.Cu") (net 16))
 (segment (start 108.62 88) (end 107 88) (width 0.2) (layer "B.Cu") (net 16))
 (segment (start 107 88) (end 100.35 81.35) (width 0.2) (layer "B.Cu") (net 16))
 (segment (start 111.73 91.11) (end 108.62 88) (width 0.2) (layer "B.Cu") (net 16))
 (segment (start 104.04 85.96) (end 102.04 85.96) (width 0.2) (layer "F.Cu") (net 15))
 (segment (start 100.35 85.35) (end 100.35 84) (width 0.2) (layer "F.Cu") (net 15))
 (segment (start 104 85.92) (end 104 83.4) (width 0.2) (layer "F.Cu") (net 15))
 (segment (start 104.04 85.96) (end 104 85.92) (width 0.2) (layer "F.Cu") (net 15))
 (segment (start 109.19 91.11) (end 104.04 85.96) (width 0.2) (layer "F.Cu") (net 15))
 (segment (start 102.04 85.96) (end 102 86) (width 0.2) (layer "F.Cu") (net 15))
 (segment (start 102 86) (end 101 86) (width 0.2) (layer "F.Cu") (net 15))
 (segment (start 101 86) (end 100.35 85.35) (width 0.2) (layer "F.Cu") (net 15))
 (segment (start 96.80795 117.272844) (end 103.30795 117.272844) (width 0.2) (layer "F.Cu") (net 14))
 (segment (start 95 115.464894) (end 96.80795 117.272844) (width 0.2) (layer "F.Cu") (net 14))
 (segment (start 95 112) (end 95 115.464894) (width 0.2) (layer "F.Cu") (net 14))
 (segment (start 88.87 108.89) (end 90.98 111) (width 0.2) (layer "F.Cu") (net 14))
 (segment (start 94 111) (end 95 112) (width 0.2) (layer "F.Cu") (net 14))
 (segment (start 90.98 111) (end 94 111) (width 0.2) (layer "F.Cu") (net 14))
 (segment (start 105.945214 117.25) (end 106.75 117.25) (width 0.2) (layer "F.Cu") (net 4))
 (segment (start 98.736214 110.041) (end 105.945214 117.25) (width 0.2) (layer "F.Cu") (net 4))
 (segment (start 106.75 117.25) (end 113.25 117.25) (width 0.2) (layer "F.Cu") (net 4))
 (segment (start 91.41 108.89) (end 92.561 110.041) (width 0.2) (layer "F.Cu") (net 4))
 (segment (start 92.561 110.041) (end 98.736214 110.041) (width 0.2) (layer "F.Cu") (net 4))
 (segment (start 99.923342 113.923342) (end 100 114) (width 0.2) (layer "F.Cu") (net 13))
 (segment (start 99.923342 112.076658) (end 99.923342 113.923342) (width 0.2) (layer "F.Cu") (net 13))
 (via (at 100 114) (size 0.6) (drill 0.3) (layers "F.Cu" "B.Cu") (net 13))
 (via (at 99.923342 112.076658) (size 0.6) (drill 0.3) (layers "F.Cu" "B.Cu") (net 13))
 (segment (start 116.75 117.25) (end 123.25 117.25) (width 0.2) (layer "B.Cu") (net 13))
 (segment (start 99.923342 111.923342) (end 99.923342 112.076658) (width 0.2) (layer "B.Cu") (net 13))
 (segment (start 101.949 115.949) (end 115.449 115.949) (width 0.2) (layer "B.Cu") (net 13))
 (segment (start 96.89 108.89) (end 99.923342 111.923342) (width 0.2) (layer "B.Cu") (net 13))
 (segment (start 115.449 115.949) (end 116.75 117.25) (width 0.2) (layer "B.Cu") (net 13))
 (segment (start 96.49 108.89) (end 96.89 108.89) (width 0.2) (layer "B.Cu") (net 13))
 (segment (start 100 114) (end 101.949 115.949) (width 0.2) (layer "B.Cu") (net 13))
 (segment (start 99.03 108.89) (end 101.589 111.449) (width 0.2) (layer "F.Cu") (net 22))
 (segment (start 120.109108 111.449) (end 125.910108 117.25) (width 0.2) (layer "F.Cu") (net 22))
 (segment (start 127 117.25) (end 133.5 117.25) (width 0.2) (layer "F.Cu") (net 22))
 (segment (start 125.910108 117.25) (end 127 117.25) (width 0.2) (layer "F.Cu") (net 22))
 (segment (start 101.589 111.449) (end 120.109108 111.449) (width 0.2) (layer "F.Cu") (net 22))
 (segment (start 108 89) (end 111 89) (width 0.2) (layer "F.Cu") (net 10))
 (via (at 111 89) (size 0.6) (drill 0.3) (layers "F.Cu" "B.Cu") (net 10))
 (via (at 108 89) (size 0.6) (drill 0.3) (layers "F.Cu" "B.Cu") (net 10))
 (segment (start 91.98 88) (end 95 88) (width 0.2) (layer "B.Cu") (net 10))
 (segment (start 95 88) (end 96 89) (width 0.2) (layer "B.Cu") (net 10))
 (segment (start 111 89) (end 127.085 89) (width 0.2) (layer "B.Cu") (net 10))
 (segment (start 96 89) (end 108 89) (width 0.2) (layer "B.Cu") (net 10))
 (segment (start 127.085 89) (end 135.815 80.27) (width 0.2) (layer "B.Cu") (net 10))
 (segment (start 88.87 91.11) (end 91.98 88) (width 0.2) (layer "B.Cu") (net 10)))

